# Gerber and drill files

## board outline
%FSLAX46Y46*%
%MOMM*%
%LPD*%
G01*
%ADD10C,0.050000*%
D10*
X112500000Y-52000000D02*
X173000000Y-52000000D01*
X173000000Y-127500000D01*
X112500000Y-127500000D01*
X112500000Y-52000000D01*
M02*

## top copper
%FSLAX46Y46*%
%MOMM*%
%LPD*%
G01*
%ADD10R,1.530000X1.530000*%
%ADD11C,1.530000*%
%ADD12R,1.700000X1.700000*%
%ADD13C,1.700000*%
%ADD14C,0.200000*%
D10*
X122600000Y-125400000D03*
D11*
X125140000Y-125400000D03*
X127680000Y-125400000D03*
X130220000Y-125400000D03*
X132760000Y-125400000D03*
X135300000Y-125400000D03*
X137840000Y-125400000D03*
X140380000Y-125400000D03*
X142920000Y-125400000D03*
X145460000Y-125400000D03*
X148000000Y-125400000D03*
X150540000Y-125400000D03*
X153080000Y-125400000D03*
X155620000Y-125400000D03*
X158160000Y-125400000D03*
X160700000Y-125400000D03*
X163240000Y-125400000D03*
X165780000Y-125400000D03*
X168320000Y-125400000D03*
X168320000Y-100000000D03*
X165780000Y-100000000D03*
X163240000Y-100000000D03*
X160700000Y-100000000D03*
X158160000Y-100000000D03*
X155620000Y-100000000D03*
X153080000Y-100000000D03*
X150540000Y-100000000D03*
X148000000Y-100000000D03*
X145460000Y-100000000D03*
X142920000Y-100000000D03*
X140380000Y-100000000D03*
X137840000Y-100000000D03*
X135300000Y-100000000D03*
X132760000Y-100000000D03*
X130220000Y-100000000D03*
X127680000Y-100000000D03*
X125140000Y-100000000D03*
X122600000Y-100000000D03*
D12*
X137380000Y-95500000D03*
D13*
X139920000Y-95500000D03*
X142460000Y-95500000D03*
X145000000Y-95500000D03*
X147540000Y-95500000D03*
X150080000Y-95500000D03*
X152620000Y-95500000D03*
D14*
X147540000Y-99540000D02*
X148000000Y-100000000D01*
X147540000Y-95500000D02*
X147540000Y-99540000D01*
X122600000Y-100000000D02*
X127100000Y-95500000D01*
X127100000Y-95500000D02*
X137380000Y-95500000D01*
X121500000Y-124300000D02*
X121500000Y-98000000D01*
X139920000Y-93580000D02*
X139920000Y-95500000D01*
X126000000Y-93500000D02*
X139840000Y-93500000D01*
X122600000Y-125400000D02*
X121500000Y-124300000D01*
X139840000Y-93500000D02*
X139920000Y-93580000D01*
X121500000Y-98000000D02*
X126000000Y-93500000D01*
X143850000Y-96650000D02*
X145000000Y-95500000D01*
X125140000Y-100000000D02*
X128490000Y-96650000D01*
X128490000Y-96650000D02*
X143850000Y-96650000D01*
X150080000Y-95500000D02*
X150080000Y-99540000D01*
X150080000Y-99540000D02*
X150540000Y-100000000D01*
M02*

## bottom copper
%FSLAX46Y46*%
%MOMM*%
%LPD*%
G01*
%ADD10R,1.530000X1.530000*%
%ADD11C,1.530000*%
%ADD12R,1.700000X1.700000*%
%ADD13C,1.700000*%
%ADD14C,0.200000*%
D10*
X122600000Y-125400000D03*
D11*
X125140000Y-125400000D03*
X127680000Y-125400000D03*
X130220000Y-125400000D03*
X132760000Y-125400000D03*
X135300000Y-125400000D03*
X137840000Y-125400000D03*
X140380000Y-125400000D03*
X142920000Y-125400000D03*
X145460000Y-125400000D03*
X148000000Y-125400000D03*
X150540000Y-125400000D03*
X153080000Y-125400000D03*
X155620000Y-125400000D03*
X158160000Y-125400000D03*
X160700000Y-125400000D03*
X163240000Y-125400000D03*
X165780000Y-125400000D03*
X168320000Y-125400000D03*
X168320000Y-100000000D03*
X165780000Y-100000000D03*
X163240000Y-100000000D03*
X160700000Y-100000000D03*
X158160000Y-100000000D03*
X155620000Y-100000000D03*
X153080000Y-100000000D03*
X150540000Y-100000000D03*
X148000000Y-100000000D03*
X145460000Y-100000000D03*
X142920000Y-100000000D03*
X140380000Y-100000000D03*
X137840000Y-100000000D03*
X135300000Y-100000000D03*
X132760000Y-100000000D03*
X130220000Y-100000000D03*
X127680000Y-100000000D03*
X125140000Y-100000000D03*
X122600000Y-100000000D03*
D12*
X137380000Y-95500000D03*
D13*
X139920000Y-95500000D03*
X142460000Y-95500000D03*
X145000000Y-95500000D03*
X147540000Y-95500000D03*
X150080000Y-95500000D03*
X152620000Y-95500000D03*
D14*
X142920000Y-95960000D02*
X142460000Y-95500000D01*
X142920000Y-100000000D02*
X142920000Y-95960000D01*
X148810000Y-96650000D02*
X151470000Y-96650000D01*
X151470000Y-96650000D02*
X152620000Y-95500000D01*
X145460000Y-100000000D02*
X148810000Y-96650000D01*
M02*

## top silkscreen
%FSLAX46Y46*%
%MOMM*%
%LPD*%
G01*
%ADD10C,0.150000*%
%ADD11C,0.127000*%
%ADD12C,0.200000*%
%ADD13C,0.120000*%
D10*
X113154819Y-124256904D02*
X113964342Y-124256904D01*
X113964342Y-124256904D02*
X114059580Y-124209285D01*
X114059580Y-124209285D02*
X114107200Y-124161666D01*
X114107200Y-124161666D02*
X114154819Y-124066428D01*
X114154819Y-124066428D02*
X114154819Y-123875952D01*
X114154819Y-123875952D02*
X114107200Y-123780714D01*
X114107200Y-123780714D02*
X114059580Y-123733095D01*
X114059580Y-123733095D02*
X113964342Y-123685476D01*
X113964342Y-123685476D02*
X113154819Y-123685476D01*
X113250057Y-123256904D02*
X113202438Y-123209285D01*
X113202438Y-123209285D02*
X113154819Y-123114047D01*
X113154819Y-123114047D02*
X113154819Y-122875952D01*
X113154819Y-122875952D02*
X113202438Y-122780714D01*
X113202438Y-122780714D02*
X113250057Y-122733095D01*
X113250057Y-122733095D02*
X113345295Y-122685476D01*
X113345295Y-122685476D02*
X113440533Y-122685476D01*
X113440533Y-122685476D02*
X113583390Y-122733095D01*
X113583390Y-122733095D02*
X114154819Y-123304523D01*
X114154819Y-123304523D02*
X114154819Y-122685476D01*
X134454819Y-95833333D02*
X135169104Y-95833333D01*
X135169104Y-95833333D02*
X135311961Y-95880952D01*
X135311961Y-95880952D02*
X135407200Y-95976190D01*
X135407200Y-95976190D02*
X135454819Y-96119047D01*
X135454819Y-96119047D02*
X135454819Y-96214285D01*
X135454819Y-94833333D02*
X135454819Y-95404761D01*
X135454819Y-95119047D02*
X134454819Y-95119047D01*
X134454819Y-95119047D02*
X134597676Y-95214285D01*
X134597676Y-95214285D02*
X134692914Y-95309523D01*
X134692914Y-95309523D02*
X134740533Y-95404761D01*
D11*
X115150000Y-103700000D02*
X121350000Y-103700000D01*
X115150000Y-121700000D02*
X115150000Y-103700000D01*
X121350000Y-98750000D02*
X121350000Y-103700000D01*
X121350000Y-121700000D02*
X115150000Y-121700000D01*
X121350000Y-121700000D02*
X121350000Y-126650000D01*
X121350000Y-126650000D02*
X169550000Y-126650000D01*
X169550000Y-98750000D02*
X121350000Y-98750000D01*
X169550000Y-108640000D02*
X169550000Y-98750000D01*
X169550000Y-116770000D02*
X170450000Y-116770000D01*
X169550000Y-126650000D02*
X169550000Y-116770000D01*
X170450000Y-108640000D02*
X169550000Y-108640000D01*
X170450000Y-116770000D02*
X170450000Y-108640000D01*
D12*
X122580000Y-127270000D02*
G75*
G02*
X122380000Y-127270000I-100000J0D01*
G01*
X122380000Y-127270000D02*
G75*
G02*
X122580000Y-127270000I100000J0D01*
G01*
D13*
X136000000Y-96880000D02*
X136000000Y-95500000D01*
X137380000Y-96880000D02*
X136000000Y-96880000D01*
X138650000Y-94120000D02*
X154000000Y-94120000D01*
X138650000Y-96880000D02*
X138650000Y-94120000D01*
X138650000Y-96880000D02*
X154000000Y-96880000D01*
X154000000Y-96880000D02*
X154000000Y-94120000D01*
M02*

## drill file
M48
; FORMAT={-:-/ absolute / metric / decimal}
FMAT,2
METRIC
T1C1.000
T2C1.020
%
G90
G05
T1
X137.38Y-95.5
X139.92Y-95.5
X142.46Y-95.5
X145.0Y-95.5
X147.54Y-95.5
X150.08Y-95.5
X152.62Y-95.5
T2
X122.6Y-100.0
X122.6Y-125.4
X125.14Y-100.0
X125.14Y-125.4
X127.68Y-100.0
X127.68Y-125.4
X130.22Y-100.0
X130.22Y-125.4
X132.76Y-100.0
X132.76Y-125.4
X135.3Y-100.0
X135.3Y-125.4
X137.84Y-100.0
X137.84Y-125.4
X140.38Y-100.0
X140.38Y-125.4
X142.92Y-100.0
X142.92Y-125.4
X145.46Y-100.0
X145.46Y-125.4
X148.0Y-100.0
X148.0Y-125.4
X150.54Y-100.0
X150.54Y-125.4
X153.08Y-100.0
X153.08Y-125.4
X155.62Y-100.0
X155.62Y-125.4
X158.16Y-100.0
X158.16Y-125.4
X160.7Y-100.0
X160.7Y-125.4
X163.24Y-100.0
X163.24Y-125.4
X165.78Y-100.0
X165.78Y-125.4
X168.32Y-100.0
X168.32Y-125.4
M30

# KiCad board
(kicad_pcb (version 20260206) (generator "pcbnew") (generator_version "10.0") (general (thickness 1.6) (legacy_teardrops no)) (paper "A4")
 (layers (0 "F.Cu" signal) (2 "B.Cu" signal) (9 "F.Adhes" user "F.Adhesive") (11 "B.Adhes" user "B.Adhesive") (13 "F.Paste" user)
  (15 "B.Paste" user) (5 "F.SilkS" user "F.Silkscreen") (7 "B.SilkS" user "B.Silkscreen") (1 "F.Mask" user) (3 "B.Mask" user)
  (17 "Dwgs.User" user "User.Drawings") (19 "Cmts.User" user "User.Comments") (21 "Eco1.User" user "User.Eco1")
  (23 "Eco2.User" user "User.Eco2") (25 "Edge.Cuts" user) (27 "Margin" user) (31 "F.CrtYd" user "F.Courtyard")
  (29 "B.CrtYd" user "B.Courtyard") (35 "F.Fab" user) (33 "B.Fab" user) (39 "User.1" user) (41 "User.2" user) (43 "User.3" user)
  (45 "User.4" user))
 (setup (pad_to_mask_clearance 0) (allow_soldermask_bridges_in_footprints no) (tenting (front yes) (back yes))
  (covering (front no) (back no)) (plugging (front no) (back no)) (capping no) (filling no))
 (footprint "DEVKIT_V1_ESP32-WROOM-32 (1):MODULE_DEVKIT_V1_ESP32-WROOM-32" (layer "F.Cu") (at 145.45 112.7 90)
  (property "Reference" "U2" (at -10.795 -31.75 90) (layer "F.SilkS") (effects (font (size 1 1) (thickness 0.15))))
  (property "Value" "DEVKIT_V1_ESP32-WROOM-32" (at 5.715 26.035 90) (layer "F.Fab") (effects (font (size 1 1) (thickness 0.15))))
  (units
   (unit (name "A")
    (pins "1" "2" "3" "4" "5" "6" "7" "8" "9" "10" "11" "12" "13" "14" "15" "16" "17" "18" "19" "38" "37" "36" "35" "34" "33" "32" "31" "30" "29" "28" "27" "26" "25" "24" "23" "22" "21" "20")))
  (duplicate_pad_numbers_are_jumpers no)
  (fp_line (start 9 -30.3) (end 9 -24.1) (stroke (width 0.127) (type solid)) (layer "F.SilkS"))
  (fp_line (start -9 -30.3) (end 9 -30.3) (stroke (width 0.127) (type solid)) (layer "F.SilkS"))
  (fp_line (start 13.95 -24.1) (end 9 -24.1) (stroke (width 0.127) (type solid)) (layer "F.SilkS"))
  (fp_line (start -9 -24.1) (end -9 -30.3) (stroke (width 0.127) (type solid)) (layer "F.SilkS"))
  (fp_line (start -9 -24.1) (end -13.95 -24.1) (stroke (width 0.127) (type solid)) (layer "F.SilkS"))
  (fp_line (start -13.95 -24.1) (end -13.95 24.1) (stroke (width 0.127) (type solid)) (layer "F.SilkS"))
  (fp_line (start 13.95 24.1) (end 13.95 -24.1) (stroke (width 0.127) (type solid)) (layer "F.SilkS"))
  (fp_line (start 4.06 24.1) (end 13.95 24.1) (stroke (width 0.127) (type solid)) (layer "F.SilkS"))
  (fp_line (start -4.07 24.1) (end -4.07 25) (stroke (width 0.127) (type solid)) (layer "F.SilkS"))
  (fp_line (start -13.95 24.1) (end -4.07 24.1) (stroke (width 0.127) (type solid)) (layer "F.SilkS"))
  (fp_line (start 4.06 25) (end 4.06 24.1) (stroke (width 0.127) (type solid)) (layer "F.SilkS"))
  (fp_line (start -4.07 25) (end 4.06 25) (stroke (width 0.127) (type solid)) (layer "F.SilkS"))
  (fp_circle (center -14.57 -22.97) (end -14.47 -22.97) (stroke (width 0.2) (type solid)) (fill no) (layer "F.SilkS"))
  (pad "1" thru_hole rect (at -12.7 -22.85 90) (size 1.53 1.53) (drill 1.02) (layers "*.Cu" "*.Mask") (remove_unused_layers no) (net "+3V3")
   (solder_mask_margin 0.102))
  (pad "2" thru_hole circle (at -12.7 -20.31 90) (size 1.53 1.53) (drill 1.02) (layers "*.Cu" "*.Mask") (remove_unused_layers no)
   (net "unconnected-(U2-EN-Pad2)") (solder_mask_margin 0.102))
  (pad "3" thru_hole circle (at -12.7 -17.77 90) (size 1.53 1.53) (drill 1.02) (layers "*.Cu" "*.Mask") (remove_unused_layers no)
   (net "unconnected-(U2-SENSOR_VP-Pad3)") (solder_mask_margin 0.102))
  (pad "4" thru_hole circle (at -12.7 -15.23 90) (size 1.53 1.53) (drill 1.02) (layers "*.Cu" "*.Mask") (remove_unused_layers no)
   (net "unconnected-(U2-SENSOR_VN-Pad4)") (solder_mask_margin 0.102))
  (pad "5" thru_hole circle (at -12.7 -12.69 90) (size 1.53 1.53) (drill 1.02) (layers "*.Cu" "*.Mask") (remove_unused_layers no)
   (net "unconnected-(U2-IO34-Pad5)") (solder_mask_margin 0.102))
  (pad "6" thru_hole circle (at -12.7 -10.15 90) (size 1.53 1.53) (drill 1.02) (layers "*.Cu" "*.Mask") (remove_unused_layers no)
   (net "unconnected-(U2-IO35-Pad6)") (solder_mask_margin 0.102))
  (pad "7" thru_hole circle (at -12.7 -7.61 90) (size 1.53 1.53) (drill 1.02) (layers "*.Cu" "*.Mask") (remove_unused_layers no)
   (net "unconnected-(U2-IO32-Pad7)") (solder_mask_margin 0.102))
  (pad "8" thru_hole circle (at -12.7 -5.07 90) (size 1.53 1.53) (drill 1.02) (layers "*.Cu" "*.Mask") (remove_unused_layers no)
   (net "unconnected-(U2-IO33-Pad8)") (solder_mask_margin 0.102))
  (pad "9" thru_hole circle (at -12.7 -2.53 90) (size 1.53 1.53) (drill 1.02) (layers "*.Cu" "*.Mask") (remove_unused_layers no)
   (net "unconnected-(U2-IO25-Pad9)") (solder_mask_margin 0.102))
  (pad "10" thru_hole circle (at -12.7 0.01 90) (size 1.53 1.53) (drill 1.02) (layers "*.Cu" "*.Mask") (remove_unused_layers no)
   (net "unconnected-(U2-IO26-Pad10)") (solder_mask_margin 0.102))
  (pad "11" thru_hole circle (at -12.7 2.55 90) (size 1.53 1.53) (drill 1.02) (layers "*.Cu" "*.Mask") (remove_unused_layers no)
   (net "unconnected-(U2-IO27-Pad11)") (solder_mask_margin 0.102))
  (pad "12" thru_hole circle (at -12.7 5.09 90) (size 1.53 1.53) (drill 1.02) (layers "*.Cu" "*.Mask") (remove_unused_layers no)
   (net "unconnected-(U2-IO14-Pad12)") (solder_mask_margin 0.102))
  (pad "13" thru_hole circle (at -12.7 7.63 90) (size 1.53 1.53) (drill 1.02) (layers "*.Cu" "*.Mask") (remove_unused_layers no)
   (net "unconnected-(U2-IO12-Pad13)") (solder_mask_margin 0.102))
  (pad "14" thru_hole circle (at -12.7 10.17 90) (size 1.53 1.53) (drill 1.02) (layers "*.Cu" "*.Mask") (remove_unused_layers no)
   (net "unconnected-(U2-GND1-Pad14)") (solder_mask_margin 0.102))
  (pad "15" thru_hole circle (at -12.7 12.71 90) (size 1.53 1.53) (drill 1.02) (layers "*.Cu" "*.Mask") (remove_unused_layers no)
   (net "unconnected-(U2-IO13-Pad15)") (solder_mask_margin 0.102))
  (pad "16" thru_hole circle (at -12.7 15.25 90) (size 1.53 1.53) (drill 1.02) (layers "*.Cu" "*.Mask") (remove_unused_layers no)
   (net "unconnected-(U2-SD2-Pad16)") (solder_mask_margin 0.102))
  (pad "17" thru_hole circle (at -12.7 17.79 90) (size 1.53 1.53) (drill 1.02) (layers "*.Cu" "*.Mask") (remove_unused_layers no)
   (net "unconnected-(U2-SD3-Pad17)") (solder_mask_margin 0.102))
  (pad "18" thru_hole circle (at -12.7 20.33 90) (size 1.53 1.53) (drill 1.02) (layers "*.Cu" "*.Mask") (remove_unused_layers no)
   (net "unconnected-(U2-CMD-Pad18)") (solder_mask_margin 0.102))
  (pad "19" thru_hole circle (at -12.7 22.87 90) (size 1.53 1.53) (drill 1.02) (layers "*.Cu" "*.Mask") (remove_unused_layers no)
   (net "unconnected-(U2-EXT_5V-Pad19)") (solder_mask_margin 0.102))
  (pad "20" thru_hole circle (at 12.7 22.87 90) (size 1.53 1.53) (drill 1.02) (layers "*.Cu" "*.Mask") (remove_unused_layers no)
   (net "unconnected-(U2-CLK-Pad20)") (solder_mask_margin 0.102))
  (pad "21" thru_hole circle (at 12.7 20.33 90) (size 1.53 1.53) (drill 1.02) (layers "*.Cu" "*.Mask") (remove_unused_layers no)
   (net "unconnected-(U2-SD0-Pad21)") (solder_mask_margin 0.102))
  (pad "22" thru_hole circle (at 12.7 17.79 90) (size 1.53 1.53) (drill 1.02) (layers "*.Cu" "*.Mask") (remove_unused_layers no)
   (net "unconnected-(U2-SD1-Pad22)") (solder_mask_margin 0.102))
  (pad "23" thru_hole circle (at 12.7 15.25 90) (size 1.53 1.53) (drill 1.02) (layers "*.Cu" "*.Mask") (remove_unused_layers no)
   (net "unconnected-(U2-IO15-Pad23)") (solder_mask_margin 0.102))
  (pad "24" thru_hole circle (at 12.7 12.71 90) (size 1.53 1.53) (drill 1.02) (layers "*.Cu" "*.Mask") (remove_unused_layers no)
   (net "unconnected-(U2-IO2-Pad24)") (solder_mask_margin 0.102))
  (pad "25" thru_hole circle (at 12.7 10.17 90) (size 1.53 1.53) (drill 1.02) (layers "*.Cu" "*.Mask") (remove_unused_layers no)
   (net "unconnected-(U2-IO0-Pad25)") (solder_mask_margin 0.102))
  (pad "26" thru_hole circle (at 12.7 7.63 90) (size 1.53 1.53) (drill 1.02) (layers "*.Cu" "*.Mask") (remove_unused_layers no)
   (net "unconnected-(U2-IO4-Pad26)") (solder_mask_margin 0.102))
  (pad "27" thru_hole circle (at 12.7 5.09 90) (size 1.53 1.53) (drill 1.02) (layers "*.Cu" "*.Mask") (remove_unused_layers no) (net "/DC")
   (solder_mask_margin 0.102))
  (pad "28" thru_hole circle (at 12.7 2.55 90) (size 1.53 1.53) (drill 1.02) (layers "*.Cu" "*.Mask") (remove_unused_layers no) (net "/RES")
   (solder_mask_margin 0.102))
  (pad "29" thru_hole circle (at 12.7 0.01 90) (size 1.53 1.53) (drill 1.02) (layers "*.Cu" "*.Mask") (remove_unused_layers no) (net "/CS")
   (solder_mask_margin 0.102))
  (pad "30" thru_hole circle (at 12.7 -2.53 90) (size 1.53 1.53) (drill 1.02) (layers "*.Cu" "*.Mask") (remove_unused_layers no)
   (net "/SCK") (solder_mask_margin 0.102))
  (pad "31" thru_hole circle (at 12.7 -5.07 90) (size 1.53 1.53) (drill 1.02) (layers "*.Cu" "*.Mask") (remove_unused_layers no)
   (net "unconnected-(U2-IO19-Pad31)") (solder_mask_margin 0.102))
  (pad "32" thru_hole circle (at 12.7 -7.61 90) (size 1.53 1.53) (drill 1.02) (layers "*.Cu" "*.Mask") (remove_unused_layers no)
   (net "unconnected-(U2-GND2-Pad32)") (solder_mask_margin 0.102))
  (pad "33" thru_hole circle (at 12.7 -10.15 90) (size 1.53 1.53) (drill 1.02) (layers "*.Cu" "*.Mask") (remove_unused_layers no)
   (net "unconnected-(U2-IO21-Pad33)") (solder_mask_margin 0.102))
  (pad "34" thru_hole circle (at 12.7 -12.69 90) (size 1.53 1.53) (drill 1.02) (layers "*.Cu" "*.Mask") (remove_unused_layers no)
   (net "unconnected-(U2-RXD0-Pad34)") (solder_mask_margin 0.102))
  (pad "35" thru_hole circle (at 12.7 -15.23 90) (size 1.53 1.53) (drill 1.02) (layers "*.Cu" "*.Mask") (remove_unused_layers no)
   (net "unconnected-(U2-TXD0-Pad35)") (solder_mask_margin 0.102))
  (pad "36" thru_hole circle (at 12.7 -17.77 90) (size 1.53 1.53) (drill 1.02) (layers "*.Cu" "*.Mask") (remove_unused_layers no)
   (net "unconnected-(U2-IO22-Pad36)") (solder_mask_margin 0.102))
  (pad "37" thru_hole circle (at 12.7 -20.31 90) (size 1.53 1.53) (drill 1.02) (layers "*.Cu" "*.Mask") (remove_unused_layers no)
   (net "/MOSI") (solder_mask_margin 0.102))
  (pad "38" thru_hole circle (at 12.7 -22.85 90) (size 1.53 1.53) (drill 1.02) (layers "*.Cu" "*.Mask") (remove_unused_layers no)
   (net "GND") (solder_mask_margin 0.102)))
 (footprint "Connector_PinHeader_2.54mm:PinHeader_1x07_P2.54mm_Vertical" (layer "F.Cu") (at 137.38 95.5 90)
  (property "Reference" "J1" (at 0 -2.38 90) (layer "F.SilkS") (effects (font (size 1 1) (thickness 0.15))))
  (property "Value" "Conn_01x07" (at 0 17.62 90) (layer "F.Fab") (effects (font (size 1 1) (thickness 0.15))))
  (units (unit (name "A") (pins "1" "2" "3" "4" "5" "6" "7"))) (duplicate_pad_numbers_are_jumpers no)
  (fp_line (start -1.38 -1.38) (end 0 -1.38) (stroke (width 0.12) (type solid)) (layer "F.SilkS"))
  (fp_line (start -1.38 0) (end -1.38 -1.38) (stroke (width 0.12) (type solid)) (layer "F.SilkS"))
  (fp_line (start 1.38 1.27) (end 1.38 16.62) (stroke (width 0.12) (type solid)) (layer "F.SilkS"))
  (fp_line (start -1.38 1.27) (end 1.38 1.27) (stroke (width 0.12) (type solid)) (layer "F.SilkS"))
  (fp_line (start -1.38 1.27) (end -1.38 16.62) (stroke (width 0.12) (type solid)) (layer "F.SilkS"))
  (fp_line (start -1.38 16.62) (end 1.38 16.62) (stroke (width 0.12) (type solid)) (layer "F.SilkS"))
  (pad "1" thru_hole rect (at 0 0 90) (size 1.7 1.7) (drill 1) (layers "*.Cu" "*.Mask") (remove_unused_layers no) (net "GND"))
  (pad "2" thru_hole circle (at 0 2.54 90) (size 1.7 1.7) (drill 1) (layers "*.Cu" "*.Mask") (remove_unused_layers no) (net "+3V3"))
  (pad "3" thru_hole circle (at 0 5.08 90) (size 1.7 1.7) (drill 1) (layers "*.Cu" "*.Mask") (remove_unused_layers no) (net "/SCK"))
  (pad "4" thru_hole circle (at 0 7.62 90) (size 1.7 1.7) (drill 1) (layers "*.Cu" "*.Mask") (remove_unused_layers no) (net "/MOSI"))
  (pad "5" thru_hole circle (at 0 10.16 90) (size 1.7 1.7) (drill 1) (layers "*.Cu" "*.Mask") (remove_unused_layers no) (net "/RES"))
  (pad "6" thru_hole circle (at 0 12.7 90) (size 1.7 1.7) (drill 1) (layers "*.Cu" "*.Mask") (remove_unused_layers no) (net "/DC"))
  (pad "7" thru_hole circle (at 0 15.24 90) (size 1.7 1.7) (drill 1) (layers "*.Cu" "*.Mask") (remove_unused_layers no) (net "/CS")))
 (gr_rect (start 112.5 52) (end 173 127.5) (stroke (width 0.05) (type default)) (fill no) (layer "Edge.Cuts"))
 (segment (start 142.92 95.96) (end 142.46 95.5) (width 0.2) (layer "B.Cu") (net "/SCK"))
 (segment (start 142.92 100) (end 142.92 95.96) (width 0.2) (layer "B.Cu") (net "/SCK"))
 (segment (start 147.54 99.54) (end 148 100) (width 0.2) (layer "F.Cu") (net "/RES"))
 (segment (start 147.54 95.5) (end 147.54 99.54) (width 0.2) (layer "F.Cu") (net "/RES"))
 (segment (start 122.6 100) (end 127.1 95.5) (width 0.2) (layer "F.Cu") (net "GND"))
 (segment (start 127.1 95.5) (end 137.38 95.5) (width 0.2) (layer "F.Cu") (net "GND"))
 (segment (start 121.5 124.3) (end 121.5 98) (width 0.2) (layer "F.Cu") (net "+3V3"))
 (segment (start 139.92 93.58) (end 139.92 95.5) (width 0.2) (layer "F.Cu") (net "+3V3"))
 (segment (start 126 93.5) (end 139.84 93.5) (width 0.2) (layer "F.Cu") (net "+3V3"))
 (segment (start 122.6 125.4) (end 121.5 124.3) (width 0.2) (layer "F.Cu") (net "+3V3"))
 (segment (start 139.84 93.5) (end 139.92 93.58) (width 0.2) (layer "F.Cu") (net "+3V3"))
 (segment (start 121.5 98) (end 126 93.5) (width 0.2) (layer "F.Cu") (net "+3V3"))
 (segment (start 143.85 96.65) (end 145 95.5) (width 0.2) (layer "F.Cu") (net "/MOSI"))
 (segment (start 125.14 100) (end 128.49 96.65) (width 0.2) (layer "F.Cu") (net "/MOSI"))
 (segment (start 128.49 96.65) (end 143.85 96.65) (width 0.2) (layer "F.Cu") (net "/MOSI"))
 (segment (start 148.81 96.65) (end 151.47 96.65) (width 0.2) (layer "B.Cu") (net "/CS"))
 (segment (start 151.47 96.65) (end 152.62 95.5) (width 0.2) (layer "B.Cu") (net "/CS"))
 (segment (start 145.46 100) (end 148.81 96.65) (width 0.2) (layer "B.Cu") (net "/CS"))
 (segment (start 150.08 95.5) (end 150.08 99.54) (width 0.2) (layer "F.Cu") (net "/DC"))
 (segment (start 150.08 99.54) (end 150.54 100) (width 0.2) (layer "F.Cu") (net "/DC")))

